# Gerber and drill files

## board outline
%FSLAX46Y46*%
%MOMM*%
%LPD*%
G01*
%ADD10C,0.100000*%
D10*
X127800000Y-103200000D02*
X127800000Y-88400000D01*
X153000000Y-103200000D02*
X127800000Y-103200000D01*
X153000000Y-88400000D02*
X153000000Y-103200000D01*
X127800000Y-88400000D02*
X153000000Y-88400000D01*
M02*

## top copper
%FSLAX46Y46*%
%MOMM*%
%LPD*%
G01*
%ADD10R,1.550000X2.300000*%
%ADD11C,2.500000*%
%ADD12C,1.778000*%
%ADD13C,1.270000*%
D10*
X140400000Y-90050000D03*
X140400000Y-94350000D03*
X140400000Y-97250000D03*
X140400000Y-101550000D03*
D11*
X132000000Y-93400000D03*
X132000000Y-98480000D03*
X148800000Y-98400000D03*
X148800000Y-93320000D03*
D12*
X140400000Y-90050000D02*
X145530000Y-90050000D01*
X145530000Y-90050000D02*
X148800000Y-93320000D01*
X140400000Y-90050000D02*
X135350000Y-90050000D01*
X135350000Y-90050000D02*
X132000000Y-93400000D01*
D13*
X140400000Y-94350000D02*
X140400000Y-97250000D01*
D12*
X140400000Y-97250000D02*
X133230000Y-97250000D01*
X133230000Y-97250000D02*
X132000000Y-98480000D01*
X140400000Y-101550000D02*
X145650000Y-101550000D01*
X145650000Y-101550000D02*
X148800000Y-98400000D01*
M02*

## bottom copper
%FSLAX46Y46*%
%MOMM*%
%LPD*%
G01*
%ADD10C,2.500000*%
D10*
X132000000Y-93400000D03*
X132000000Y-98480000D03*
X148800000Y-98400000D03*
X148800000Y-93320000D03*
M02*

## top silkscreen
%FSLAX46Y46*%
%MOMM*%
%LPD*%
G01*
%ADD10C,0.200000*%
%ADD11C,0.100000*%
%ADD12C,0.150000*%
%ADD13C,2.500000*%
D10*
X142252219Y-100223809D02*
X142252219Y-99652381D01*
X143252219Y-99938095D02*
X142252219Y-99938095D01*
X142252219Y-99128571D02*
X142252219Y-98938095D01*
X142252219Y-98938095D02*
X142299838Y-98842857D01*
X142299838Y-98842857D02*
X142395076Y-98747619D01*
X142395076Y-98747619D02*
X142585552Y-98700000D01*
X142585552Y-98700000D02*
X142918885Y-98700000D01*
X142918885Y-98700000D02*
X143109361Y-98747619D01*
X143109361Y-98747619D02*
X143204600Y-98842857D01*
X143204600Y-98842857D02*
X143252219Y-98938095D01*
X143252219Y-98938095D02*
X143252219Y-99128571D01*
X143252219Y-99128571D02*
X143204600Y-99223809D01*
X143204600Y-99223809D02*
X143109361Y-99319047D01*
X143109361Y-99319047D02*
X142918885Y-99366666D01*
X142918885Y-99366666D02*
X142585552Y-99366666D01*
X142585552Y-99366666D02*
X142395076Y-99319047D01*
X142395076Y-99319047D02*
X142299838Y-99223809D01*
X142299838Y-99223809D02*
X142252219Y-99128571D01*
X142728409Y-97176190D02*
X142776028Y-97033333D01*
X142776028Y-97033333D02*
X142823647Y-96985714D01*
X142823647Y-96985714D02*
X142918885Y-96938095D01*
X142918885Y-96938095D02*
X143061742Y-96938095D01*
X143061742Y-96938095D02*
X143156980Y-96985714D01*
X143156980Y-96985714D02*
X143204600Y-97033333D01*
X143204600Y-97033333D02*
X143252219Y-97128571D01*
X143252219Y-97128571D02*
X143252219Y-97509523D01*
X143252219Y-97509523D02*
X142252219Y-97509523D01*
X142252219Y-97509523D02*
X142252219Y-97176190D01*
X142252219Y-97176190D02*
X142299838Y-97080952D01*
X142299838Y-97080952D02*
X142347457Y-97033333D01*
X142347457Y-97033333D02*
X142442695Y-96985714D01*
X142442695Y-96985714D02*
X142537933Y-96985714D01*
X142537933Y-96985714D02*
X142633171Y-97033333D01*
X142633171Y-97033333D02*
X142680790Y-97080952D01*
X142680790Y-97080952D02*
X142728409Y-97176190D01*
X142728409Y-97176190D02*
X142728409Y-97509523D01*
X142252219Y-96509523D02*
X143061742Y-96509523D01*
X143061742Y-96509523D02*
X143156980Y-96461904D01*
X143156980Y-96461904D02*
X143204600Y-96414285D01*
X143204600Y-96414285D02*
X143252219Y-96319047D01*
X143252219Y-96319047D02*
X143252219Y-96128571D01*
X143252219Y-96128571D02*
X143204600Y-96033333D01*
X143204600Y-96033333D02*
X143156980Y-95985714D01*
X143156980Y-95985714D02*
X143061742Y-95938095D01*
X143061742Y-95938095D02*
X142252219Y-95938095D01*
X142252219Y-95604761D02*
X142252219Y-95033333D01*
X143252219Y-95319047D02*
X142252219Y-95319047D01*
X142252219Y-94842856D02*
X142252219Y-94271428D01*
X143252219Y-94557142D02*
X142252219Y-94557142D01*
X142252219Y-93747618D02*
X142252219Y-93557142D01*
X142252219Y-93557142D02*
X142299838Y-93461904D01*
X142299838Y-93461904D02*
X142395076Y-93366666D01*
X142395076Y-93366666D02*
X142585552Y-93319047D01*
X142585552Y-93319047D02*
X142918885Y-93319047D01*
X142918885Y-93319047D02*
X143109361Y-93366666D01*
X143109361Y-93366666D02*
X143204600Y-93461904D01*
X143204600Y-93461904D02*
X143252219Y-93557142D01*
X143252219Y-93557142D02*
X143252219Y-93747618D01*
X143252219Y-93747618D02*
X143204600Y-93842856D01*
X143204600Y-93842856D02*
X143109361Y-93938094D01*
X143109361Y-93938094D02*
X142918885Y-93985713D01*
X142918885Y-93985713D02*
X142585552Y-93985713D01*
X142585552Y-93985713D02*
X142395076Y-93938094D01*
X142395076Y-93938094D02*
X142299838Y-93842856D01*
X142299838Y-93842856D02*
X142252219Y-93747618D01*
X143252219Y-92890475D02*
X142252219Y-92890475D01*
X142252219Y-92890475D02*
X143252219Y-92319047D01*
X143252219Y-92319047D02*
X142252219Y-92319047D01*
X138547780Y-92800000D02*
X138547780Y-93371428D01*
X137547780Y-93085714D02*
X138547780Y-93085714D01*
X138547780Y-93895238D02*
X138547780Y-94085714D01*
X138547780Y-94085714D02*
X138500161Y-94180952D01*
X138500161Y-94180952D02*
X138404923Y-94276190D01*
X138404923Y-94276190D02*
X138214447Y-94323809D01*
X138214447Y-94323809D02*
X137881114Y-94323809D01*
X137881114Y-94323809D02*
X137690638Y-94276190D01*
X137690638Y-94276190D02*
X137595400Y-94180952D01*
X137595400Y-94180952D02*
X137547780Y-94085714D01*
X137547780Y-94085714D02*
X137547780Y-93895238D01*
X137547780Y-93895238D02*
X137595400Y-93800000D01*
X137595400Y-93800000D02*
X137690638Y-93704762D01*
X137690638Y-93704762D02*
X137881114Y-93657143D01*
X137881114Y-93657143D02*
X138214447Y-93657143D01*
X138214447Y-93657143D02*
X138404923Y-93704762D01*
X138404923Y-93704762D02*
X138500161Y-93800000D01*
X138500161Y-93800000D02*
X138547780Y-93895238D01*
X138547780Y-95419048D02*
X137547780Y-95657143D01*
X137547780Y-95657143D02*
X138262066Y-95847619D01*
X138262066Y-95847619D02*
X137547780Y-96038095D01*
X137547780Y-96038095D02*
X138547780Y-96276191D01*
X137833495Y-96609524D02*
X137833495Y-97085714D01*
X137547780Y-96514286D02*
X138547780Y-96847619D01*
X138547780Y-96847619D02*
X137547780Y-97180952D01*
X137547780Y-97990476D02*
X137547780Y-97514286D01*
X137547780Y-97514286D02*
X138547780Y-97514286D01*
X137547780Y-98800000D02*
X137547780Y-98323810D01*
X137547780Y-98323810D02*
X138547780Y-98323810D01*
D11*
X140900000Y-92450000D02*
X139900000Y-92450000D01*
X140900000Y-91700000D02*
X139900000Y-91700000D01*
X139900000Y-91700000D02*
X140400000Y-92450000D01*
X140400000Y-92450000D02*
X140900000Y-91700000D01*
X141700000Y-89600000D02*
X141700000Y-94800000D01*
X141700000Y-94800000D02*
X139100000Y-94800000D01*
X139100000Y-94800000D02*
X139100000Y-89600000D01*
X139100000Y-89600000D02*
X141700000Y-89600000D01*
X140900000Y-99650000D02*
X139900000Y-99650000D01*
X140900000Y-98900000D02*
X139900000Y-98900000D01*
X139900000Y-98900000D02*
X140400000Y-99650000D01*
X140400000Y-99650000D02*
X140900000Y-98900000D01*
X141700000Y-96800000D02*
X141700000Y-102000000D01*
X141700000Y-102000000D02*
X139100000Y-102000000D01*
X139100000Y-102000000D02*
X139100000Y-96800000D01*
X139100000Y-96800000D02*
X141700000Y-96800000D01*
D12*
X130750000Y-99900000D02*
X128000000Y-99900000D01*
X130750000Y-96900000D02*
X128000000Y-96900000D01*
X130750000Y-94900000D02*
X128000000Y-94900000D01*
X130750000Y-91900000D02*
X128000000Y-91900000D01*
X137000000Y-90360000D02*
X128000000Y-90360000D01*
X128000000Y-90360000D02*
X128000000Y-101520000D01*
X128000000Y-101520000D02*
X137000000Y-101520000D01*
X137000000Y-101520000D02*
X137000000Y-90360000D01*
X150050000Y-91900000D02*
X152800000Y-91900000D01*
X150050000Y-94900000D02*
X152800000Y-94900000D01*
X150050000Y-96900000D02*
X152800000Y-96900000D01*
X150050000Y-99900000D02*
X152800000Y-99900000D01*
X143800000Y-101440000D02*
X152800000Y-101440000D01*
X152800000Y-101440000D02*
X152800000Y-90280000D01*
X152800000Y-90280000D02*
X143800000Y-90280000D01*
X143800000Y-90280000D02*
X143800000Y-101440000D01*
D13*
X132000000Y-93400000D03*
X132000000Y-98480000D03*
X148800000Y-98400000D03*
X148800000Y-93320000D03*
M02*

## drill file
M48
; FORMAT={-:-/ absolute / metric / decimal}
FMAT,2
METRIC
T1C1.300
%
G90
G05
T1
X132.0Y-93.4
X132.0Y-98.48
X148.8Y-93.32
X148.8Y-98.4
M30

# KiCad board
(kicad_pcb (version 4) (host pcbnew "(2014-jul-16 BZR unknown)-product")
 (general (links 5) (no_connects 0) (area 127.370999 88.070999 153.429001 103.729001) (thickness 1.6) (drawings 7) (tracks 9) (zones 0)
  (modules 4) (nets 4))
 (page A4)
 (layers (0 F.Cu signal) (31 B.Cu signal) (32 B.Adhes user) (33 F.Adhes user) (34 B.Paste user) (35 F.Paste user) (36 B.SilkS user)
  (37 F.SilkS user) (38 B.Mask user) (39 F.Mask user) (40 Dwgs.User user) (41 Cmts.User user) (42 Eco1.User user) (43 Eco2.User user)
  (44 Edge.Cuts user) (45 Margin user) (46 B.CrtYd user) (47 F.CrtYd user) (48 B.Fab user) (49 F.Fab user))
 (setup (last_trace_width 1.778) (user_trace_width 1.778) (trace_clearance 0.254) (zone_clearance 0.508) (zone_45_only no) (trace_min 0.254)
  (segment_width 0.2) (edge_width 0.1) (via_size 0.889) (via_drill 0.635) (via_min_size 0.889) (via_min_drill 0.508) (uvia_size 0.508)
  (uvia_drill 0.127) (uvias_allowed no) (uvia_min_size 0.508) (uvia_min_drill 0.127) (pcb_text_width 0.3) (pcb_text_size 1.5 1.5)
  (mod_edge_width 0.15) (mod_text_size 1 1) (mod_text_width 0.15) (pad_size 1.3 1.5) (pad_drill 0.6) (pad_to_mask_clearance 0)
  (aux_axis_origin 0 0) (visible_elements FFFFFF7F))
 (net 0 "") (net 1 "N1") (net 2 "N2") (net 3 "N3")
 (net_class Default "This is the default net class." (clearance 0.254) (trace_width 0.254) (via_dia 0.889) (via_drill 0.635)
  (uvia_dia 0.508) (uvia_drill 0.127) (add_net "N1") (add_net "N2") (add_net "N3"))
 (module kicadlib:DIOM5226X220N (layer F.Cu) (at 140.4 92.2 270)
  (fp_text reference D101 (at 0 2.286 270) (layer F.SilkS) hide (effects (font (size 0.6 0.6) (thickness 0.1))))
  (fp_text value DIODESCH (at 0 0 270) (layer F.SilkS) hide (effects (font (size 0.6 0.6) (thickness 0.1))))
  (fp_line (start 0.25 -0.5) (end 0.25 0.5) (layer F.SilkS) (width 0.1))
  (fp_line (start -0.5 -0.5) (end -0.5 0.5) (layer F.SilkS) (width 0.1))
  (fp_line (start -0.5 0.5) (end 0.25 0) (layer F.SilkS) (width 0.1))
  (fp_line (start 0.25 0) (end -0.5 -0.5) (layer F.SilkS) (width 0.1))
  (fp_line (start -2.6 -1.3) (end 2.6 -1.3) (layer F.SilkS) (width 0.1))
  (fp_line (start 2.6 -1.3) (end 2.6 1.3) (layer F.SilkS) (width 0.1))
  (fp_line (start 2.6 1.3) (end -2.6 1.3) (layer F.SilkS) (width 0.1))
  (fp_line (start -2.6 1.3) (end -2.6 -1.3) (layer F.SilkS) (width 0.1))
  (pad 1 smd rect (at -2.15 0 270) (size 2.3 1.55) (layers F.Cu F.Paste F.Mask) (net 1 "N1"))
  (pad 2 smd rect (at 2.15 0 270) (size 2.3 1.55) (layers F.Cu F.Paste F.Mask) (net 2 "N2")))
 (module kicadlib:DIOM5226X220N (layer F.Cu) (at 140.4 99.4 270)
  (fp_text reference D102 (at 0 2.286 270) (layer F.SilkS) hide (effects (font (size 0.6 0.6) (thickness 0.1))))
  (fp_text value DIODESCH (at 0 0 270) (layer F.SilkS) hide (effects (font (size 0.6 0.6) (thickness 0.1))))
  (fp_line (start 0.25 -0.5) (end 0.25 0.5) (layer F.SilkS) (width 0.1))
  (fp_line (start -0.5 -0.5) (end -0.5 0.5) (layer F.SilkS) (width 0.1))
  (fp_line (start -0.5 0.5) (end 0.25 0) (layer F.SilkS) (width 0.1))
  (fp_line (start 0.25 0) (end -0.5 -0.5) (layer F.SilkS) (width 0.1))
  (fp_line (start -2.6 -1.3) (end 2.6 -1.3) (layer F.SilkS) (width 0.1))
  (fp_line (start 2.6 -1.3) (end 2.6 1.3) (layer F.SilkS) (width 0.1))
  (fp_line (start 2.6 1.3) (end -2.6 1.3) (layer F.SilkS) (width 0.1))
  (fp_line (start -2.6 1.3) (end -2.6 -1.3) (layer F.SilkS) (width 0.1))
  (pad 1 smd rect (at -2.15 0 270) (size 2.3 1.55) (layers F.Cu F.Paste F.Mask) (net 2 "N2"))
  (pad 2 smd rect (at 2.15 0 270) (size 2.3 1.55) (layers F.Cu F.Paste F.Mask) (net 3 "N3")))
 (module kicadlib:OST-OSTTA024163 (layer F.Cu) (at 132 93.4 270)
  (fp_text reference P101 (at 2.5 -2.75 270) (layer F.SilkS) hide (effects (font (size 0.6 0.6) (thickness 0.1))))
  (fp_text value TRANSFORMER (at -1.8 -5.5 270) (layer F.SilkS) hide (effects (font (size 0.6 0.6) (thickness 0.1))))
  (fp_line (start 6.5 1.25) (end 6.5 4) (layer F.SilkS) (width 0.15))
  (fp_line (start 3.5 1.25) (end 3.5 4) (layer F.SilkS) (width 0.15))
  (fp_line (start 1.5 1.25) (end 1.5 4) (layer F.SilkS) (width 0.15))
  (fp_line (start -1.5 1.25) (end -1.5 4) (layer F.SilkS) (width 0.15))
  (fp_line (start -3.04 -5) (end -3.04 4) (layer F.SilkS) (width 0.15))
  (fp_line (start -3.04 4) (end 8.12 4) (layer F.SilkS) (width 0.15))
  (fp_line (start 8.12 4) (end 8.12 -5) (layer F.SilkS) (width 0.15))
  (fp_line (start 8.12 -5) (end -3.04 -5) (layer F.SilkS) (width 0.15))
  (pad 1 thru_hole circle (at 0 0 270) (size 2.5 2.5) (drill 1.3) (layers *.Cu *.Mask F.SilkS) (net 1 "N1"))
  (pad 2 thru_hole circle (at 5.08 0 270) (size 2.5 2.5) (drill 1.3) (layers *.Cu *.Mask F.SilkS) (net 2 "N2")))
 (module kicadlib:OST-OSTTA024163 (layer F.Cu) (at 148.8 98.4 90)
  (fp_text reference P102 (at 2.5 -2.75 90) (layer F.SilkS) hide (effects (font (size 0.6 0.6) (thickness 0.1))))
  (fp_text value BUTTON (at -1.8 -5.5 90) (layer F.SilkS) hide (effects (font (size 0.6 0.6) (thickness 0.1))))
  (fp_line (start 6.5 1.25) (end 6.5 4) (layer F.SilkS) (width 0.15))
  (fp_line (start 3.5 1.25) (end 3.5 4) (layer F.SilkS) (width 0.15))
  (fp_line (start 1.5 1.25) (end 1.5 4) (layer F.SilkS) (width 0.15))
  (fp_line (start -1.5 1.25) (end -1.5 4) (layer F.SilkS) (width 0.15))
  (fp_line (start -3.04 -5) (end -3.04 4) (layer F.SilkS) (width 0.15))
  (fp_line (start -3.04 4) (end 8.12 4) (layer F.SilkS) (width 0.15))
  (fp_line (start 8.12 4) (end 8.12 -5) (layer F.SilkS) (width 0.15))
  (fp_line (start 8.12 -5) (end -3.04 -5) (layer F.SilkS) (width 0.15))
  (pad 1 thru_hole circle (at 0 0 90) (size 2.5 2.5) (drill 1.3) (layers *.Cu *.Mask F.SilkS) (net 3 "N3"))
  (pad 2 thru_hole circle (at 5.08 0 90) (size 2.5 2.5) (drill 1.3) (layers *.Cu *.Mask F.SilkS) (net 1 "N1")))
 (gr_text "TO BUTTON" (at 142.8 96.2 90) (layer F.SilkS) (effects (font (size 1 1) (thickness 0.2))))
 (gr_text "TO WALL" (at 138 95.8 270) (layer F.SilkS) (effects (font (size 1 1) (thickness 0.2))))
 (gr_line (start 127.8 103.2) (end 127.8 88.4) (angle 90) (layer Edge.Cuts) (width 0.1))
 (gr_line (start 153 103.2) (end 127.8 103.2) (angle 90) (layer Edge.Cuts) (width 0.1))
 (gr_line (start 153 88.4) (end 153 103.2) (angle 90) (layer Edge.Cuts) (width 0.1))
 (gr_line (start 127.8 88.4) (end 153 88.4) (angle 90) (layer Edge.Cuts) (width 0.1))
 (segment (start 140.4 90.05) (end 145.53 90.05) (width 1.778) (layer F.Cu) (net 1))
 (segment (start 145.53 90.05) (end 148.8 93.32) (width 1.778) (layer F.Cu) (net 1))
 (segment (start 140.4 90.05) (end 135.35 90.05) (width 1.778) (layer F.Cu) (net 1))
 (segment (start 135.35 90.05) (end 132 93.4) (width 1.778) (layer F.Cu) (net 1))
 (segment (start 140.4 94.35) (end 140.4 97.25) (width 1.27) (layer F.Cu) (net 2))
 (segment (start 140.4 97.25) (end 133.23 97.25) (width 1.778) (layer F.Cu) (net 2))
 (segment (start 133.23 97.25) (end 132 98.48) (width 1.778) (layer F.Cu) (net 2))
 (segment (start 140.4 101.55) (end 145.65 101.55) (width 1.778) (layer F.Cu) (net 3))
 (segment (start 145.65 101.55) (end 148.8 98.4) (width 1.778) (layer F.Cu) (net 3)))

